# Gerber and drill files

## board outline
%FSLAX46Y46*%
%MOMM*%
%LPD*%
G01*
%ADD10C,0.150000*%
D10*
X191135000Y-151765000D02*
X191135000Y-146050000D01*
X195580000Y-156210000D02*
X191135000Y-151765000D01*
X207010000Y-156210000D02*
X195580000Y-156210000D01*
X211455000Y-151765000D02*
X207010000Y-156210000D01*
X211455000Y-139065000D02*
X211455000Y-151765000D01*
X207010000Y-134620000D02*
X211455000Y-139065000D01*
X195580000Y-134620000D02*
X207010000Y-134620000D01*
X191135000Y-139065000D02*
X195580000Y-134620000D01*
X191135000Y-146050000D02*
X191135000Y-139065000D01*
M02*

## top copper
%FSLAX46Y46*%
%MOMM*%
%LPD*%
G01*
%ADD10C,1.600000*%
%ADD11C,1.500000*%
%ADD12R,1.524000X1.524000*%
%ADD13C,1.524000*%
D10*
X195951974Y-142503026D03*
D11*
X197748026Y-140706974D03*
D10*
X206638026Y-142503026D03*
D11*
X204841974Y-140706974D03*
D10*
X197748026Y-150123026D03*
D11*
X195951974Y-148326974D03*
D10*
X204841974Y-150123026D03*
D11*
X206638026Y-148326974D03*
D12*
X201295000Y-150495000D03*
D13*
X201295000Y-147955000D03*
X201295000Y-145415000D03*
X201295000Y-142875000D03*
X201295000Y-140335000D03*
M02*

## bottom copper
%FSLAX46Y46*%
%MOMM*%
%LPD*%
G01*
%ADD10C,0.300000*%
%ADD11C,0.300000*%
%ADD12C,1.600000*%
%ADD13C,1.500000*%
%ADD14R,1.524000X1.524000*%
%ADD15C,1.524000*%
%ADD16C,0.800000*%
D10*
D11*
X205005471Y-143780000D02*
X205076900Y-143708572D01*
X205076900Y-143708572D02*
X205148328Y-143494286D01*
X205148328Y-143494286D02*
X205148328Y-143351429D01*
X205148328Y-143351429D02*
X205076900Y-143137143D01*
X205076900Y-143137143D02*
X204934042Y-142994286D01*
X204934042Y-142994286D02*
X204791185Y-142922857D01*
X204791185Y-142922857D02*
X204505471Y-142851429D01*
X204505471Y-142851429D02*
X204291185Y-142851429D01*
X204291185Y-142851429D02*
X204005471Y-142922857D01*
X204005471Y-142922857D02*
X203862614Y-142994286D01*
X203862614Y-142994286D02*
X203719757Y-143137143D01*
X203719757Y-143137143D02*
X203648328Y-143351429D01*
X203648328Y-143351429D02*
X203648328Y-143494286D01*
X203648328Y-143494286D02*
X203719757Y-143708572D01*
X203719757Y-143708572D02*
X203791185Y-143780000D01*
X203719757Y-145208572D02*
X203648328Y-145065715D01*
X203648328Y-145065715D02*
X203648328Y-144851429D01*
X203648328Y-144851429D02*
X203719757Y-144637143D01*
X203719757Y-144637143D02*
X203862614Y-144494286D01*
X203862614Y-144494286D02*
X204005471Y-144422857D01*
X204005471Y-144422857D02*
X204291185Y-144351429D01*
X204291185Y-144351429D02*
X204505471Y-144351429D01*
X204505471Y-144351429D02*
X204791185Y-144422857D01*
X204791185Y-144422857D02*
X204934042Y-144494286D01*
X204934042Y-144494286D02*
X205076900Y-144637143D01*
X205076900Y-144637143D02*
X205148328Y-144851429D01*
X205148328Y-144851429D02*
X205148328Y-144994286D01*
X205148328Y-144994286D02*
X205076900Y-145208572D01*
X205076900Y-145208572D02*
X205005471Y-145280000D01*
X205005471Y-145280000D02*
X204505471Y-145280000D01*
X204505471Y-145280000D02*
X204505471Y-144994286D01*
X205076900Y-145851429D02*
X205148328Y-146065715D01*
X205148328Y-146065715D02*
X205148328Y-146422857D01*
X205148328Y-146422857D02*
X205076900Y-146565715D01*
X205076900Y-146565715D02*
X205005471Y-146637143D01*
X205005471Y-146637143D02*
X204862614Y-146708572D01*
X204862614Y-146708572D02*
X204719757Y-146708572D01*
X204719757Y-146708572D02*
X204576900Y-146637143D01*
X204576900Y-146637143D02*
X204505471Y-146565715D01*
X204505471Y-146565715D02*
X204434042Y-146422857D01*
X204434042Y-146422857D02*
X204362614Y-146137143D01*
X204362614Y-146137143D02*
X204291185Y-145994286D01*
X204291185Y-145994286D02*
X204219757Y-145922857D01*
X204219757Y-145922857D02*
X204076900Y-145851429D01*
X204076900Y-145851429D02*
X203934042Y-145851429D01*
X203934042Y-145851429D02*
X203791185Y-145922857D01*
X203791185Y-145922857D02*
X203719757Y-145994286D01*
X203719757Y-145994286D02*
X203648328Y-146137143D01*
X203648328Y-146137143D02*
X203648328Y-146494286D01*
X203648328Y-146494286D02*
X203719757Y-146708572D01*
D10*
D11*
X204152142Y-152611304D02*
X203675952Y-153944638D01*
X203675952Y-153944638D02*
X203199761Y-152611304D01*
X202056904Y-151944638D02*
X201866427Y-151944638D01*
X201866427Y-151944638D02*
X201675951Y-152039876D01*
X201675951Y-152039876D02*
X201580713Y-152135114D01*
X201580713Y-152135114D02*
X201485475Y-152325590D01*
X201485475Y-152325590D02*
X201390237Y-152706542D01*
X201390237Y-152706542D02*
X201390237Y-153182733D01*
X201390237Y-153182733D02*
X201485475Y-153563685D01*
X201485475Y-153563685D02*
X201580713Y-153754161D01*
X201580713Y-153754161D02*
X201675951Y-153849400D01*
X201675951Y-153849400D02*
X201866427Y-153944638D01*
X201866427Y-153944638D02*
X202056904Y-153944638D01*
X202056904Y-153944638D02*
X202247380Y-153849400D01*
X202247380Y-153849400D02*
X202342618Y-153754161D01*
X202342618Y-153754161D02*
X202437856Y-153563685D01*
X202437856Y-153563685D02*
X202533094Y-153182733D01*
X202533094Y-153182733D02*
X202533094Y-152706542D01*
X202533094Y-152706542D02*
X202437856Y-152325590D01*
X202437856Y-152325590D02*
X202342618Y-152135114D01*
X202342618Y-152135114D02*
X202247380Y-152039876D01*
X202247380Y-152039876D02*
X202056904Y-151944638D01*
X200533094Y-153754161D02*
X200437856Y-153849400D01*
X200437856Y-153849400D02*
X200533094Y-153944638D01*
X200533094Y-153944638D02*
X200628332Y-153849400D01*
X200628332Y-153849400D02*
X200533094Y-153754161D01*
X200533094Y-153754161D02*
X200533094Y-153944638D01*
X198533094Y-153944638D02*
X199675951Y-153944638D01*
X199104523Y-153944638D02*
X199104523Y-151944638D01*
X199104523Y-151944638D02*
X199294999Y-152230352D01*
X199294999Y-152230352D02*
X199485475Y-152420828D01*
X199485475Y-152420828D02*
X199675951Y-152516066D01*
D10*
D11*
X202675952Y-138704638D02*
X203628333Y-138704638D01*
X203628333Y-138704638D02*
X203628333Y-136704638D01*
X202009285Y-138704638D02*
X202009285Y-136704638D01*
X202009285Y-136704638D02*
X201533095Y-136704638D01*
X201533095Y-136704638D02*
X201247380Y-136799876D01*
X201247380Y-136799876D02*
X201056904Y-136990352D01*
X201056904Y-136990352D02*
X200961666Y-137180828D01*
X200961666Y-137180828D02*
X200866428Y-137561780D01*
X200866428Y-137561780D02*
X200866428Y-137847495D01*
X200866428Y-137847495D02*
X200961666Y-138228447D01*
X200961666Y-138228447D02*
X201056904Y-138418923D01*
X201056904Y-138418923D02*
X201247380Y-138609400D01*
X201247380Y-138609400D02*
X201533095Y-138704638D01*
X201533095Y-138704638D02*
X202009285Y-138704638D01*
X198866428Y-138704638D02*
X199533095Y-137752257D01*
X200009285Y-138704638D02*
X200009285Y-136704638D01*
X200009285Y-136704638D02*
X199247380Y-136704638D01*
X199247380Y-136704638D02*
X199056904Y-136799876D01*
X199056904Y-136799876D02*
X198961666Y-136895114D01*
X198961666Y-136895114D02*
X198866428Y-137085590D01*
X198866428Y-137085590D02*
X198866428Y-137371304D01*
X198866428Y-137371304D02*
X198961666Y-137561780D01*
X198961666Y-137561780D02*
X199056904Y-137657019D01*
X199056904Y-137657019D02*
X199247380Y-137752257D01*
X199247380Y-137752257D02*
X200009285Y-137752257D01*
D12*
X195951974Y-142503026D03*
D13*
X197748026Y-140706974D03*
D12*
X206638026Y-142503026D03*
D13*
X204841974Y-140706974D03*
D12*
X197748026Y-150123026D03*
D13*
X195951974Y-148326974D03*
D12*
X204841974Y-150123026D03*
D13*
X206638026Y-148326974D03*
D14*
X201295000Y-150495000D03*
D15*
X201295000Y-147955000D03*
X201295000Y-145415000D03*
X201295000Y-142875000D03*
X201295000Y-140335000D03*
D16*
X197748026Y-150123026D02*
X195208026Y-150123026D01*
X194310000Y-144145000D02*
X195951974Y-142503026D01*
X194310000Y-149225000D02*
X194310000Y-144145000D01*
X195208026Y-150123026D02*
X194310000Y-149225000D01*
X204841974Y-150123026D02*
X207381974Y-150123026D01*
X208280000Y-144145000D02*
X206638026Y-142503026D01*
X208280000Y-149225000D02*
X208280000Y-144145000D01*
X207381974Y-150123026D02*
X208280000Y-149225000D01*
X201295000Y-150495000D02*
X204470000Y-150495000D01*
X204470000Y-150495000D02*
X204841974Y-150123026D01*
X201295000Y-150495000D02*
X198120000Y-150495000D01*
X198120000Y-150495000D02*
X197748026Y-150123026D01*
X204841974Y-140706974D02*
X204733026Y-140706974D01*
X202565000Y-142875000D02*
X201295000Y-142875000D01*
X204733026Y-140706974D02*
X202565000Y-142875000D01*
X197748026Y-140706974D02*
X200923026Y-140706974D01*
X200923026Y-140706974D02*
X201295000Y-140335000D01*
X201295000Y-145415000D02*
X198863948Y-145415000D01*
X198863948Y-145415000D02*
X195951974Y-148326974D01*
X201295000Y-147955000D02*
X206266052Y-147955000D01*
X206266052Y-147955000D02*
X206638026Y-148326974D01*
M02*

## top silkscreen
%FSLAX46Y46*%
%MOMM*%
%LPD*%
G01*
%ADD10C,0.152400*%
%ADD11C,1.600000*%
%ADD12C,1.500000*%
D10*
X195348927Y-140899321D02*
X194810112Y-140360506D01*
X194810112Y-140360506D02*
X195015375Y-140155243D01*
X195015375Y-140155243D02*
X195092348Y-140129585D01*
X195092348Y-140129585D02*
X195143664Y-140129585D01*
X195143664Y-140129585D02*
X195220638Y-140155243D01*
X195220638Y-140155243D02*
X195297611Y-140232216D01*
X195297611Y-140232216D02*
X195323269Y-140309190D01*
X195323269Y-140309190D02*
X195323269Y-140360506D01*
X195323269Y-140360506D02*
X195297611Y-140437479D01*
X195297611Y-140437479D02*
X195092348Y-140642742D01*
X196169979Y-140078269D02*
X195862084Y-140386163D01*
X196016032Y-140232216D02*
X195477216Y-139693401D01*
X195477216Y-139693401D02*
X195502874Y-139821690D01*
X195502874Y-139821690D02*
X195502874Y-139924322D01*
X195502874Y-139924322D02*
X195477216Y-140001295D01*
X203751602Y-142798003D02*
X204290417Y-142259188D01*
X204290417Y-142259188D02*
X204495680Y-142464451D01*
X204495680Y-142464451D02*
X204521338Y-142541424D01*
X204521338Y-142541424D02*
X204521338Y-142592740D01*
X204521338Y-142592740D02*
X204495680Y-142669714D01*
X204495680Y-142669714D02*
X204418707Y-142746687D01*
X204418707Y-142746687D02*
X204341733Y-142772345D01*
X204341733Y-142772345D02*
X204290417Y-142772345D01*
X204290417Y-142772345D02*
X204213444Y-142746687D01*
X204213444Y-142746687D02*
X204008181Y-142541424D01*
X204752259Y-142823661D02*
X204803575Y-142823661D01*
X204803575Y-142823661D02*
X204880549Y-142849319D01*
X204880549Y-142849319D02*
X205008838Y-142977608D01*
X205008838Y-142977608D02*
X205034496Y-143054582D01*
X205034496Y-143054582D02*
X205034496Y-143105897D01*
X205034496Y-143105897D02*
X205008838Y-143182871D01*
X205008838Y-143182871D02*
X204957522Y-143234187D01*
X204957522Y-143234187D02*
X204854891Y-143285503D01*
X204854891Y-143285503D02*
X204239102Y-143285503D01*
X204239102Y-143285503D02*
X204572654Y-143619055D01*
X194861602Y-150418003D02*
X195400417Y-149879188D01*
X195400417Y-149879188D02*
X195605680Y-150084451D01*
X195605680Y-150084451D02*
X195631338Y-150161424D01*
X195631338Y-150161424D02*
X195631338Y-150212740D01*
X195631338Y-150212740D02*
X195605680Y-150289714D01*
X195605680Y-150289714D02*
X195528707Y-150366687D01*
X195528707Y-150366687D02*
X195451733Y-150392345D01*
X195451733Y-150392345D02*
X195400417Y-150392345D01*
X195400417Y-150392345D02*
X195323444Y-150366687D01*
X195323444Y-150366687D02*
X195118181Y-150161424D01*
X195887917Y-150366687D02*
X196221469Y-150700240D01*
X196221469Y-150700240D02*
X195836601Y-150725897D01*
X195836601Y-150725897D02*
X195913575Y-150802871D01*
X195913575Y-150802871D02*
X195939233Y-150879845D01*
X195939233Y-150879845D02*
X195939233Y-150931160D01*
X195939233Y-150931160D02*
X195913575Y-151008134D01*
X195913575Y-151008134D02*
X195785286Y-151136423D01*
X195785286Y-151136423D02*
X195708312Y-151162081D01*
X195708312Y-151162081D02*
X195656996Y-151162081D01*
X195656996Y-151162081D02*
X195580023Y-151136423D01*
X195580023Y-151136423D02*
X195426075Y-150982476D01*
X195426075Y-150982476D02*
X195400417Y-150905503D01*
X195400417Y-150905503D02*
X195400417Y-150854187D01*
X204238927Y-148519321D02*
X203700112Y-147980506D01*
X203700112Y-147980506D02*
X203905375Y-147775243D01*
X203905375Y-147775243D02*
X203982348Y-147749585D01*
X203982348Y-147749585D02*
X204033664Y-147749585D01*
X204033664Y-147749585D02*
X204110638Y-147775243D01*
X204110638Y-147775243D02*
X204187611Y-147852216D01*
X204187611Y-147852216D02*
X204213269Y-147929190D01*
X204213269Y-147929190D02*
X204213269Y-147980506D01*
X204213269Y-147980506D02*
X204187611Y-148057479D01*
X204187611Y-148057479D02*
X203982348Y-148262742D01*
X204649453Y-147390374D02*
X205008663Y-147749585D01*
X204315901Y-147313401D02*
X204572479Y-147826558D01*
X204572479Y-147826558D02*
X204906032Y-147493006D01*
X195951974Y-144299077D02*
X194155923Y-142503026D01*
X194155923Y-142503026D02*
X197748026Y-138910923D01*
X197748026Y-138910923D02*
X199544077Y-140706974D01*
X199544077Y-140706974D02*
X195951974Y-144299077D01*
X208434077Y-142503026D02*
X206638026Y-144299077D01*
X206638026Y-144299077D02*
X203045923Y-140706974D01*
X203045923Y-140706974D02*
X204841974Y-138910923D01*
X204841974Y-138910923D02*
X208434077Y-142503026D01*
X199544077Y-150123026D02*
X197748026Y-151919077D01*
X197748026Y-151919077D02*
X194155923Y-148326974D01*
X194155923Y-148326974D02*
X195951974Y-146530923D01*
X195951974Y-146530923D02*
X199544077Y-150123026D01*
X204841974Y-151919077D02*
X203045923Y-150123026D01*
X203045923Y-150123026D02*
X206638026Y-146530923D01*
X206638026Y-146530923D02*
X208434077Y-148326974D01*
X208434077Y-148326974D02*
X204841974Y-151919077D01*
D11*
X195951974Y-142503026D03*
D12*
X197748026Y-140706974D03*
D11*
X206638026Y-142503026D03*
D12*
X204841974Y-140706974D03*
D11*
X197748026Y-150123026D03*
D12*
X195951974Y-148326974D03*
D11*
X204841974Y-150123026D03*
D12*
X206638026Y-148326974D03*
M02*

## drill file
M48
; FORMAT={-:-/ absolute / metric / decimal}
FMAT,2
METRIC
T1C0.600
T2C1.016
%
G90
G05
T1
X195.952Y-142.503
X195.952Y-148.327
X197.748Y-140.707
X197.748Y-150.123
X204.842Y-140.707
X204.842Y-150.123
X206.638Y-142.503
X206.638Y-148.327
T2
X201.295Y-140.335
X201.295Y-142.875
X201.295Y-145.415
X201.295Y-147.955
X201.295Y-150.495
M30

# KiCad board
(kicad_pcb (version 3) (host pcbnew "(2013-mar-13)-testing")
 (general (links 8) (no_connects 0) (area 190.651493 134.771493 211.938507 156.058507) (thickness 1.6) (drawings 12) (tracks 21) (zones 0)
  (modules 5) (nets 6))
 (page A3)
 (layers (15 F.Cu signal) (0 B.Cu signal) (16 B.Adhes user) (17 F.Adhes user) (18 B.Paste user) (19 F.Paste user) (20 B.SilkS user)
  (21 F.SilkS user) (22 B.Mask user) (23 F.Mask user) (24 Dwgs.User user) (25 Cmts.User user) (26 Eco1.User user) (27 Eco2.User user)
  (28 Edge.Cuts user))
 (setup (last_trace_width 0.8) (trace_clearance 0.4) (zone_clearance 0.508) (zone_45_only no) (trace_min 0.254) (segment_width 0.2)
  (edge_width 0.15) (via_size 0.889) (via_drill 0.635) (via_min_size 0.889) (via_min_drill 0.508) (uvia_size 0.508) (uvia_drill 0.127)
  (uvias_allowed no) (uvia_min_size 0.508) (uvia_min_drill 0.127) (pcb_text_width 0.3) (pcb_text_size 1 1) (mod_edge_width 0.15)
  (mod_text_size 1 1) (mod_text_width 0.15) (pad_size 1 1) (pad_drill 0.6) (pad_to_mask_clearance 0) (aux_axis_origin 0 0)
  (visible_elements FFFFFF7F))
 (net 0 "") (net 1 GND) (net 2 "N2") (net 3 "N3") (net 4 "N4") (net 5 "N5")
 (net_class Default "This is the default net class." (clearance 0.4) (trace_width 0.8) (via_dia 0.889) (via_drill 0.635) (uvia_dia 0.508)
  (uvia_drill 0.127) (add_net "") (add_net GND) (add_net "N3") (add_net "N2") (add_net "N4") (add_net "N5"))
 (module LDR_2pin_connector (layer F.Cu) (at 196.85 141.605 45)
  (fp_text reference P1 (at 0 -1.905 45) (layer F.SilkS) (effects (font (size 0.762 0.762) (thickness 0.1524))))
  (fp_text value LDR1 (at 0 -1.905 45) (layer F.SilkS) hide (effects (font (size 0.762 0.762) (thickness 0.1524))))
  (fp_line (start -2.54 1.27) (end -2.54 -1.27) (layer F.SilkS) (width 0.1524))
  (fp_line (start -2.54 -1.27) (end 2.54 -1.27) (layer F.SilkS) (width 0.1524))
  (fp_line (start 2.54 -1.27) (end 2.54 1.27) (layer F.SilkS) (width 0.1524))
  (fp_line (start 2.54 1.27) (end -2.54 1.27) (layer F.SilkS) (width 0.1524))
  (pad 1 thru_hole circle (at -1.27 0 45) (size 1.6 1.6) (drill 0.6) (layers *.Cu *.Mask F.SilkS) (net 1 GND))
  (pad 2 thru_hole circle (at 1.27 0 45) (size 1.5 1.5) (drill 0.6) (layers *.Cu *.Mask F.SilkS) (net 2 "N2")))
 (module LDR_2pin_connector (layer F.Cu) (at 205.74 141.605 135)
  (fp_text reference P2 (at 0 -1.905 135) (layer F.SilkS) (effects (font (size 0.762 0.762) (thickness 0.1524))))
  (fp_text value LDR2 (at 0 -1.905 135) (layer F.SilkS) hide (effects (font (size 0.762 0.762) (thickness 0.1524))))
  (fp_line (start -2.54 1.27) (end -2.54 -1.27) (layer F.SilkS) (width 0.1524))
  (fp_line (start -2.54 -1.27) (end 2.54 -1.27) (layer F.SilkS) (width 0.1524))
  (fp_line (start 2.54 -1.27) (end 2.54 1.27) (layer F.SilkS) (width 0.1524))
  (fp_line (start 2.54 1.27) (end -2.54 1.27) (layer F.SilkS) (width 0.1524))
  (pad 1 thru_hole circle (at -1.27 0 135) (size 1.6 1.6) (drill 0.6) (layers *.Cu *.Mask F.SilkS) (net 1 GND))
  (pad 2 thru_hole circle (at 1.27 0 135) (size 1.5 1.5) (drill 0.6) (layers *.Cu *.Mask F.SilkS) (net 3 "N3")))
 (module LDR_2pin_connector (layer F.Cu) (at 196.85 149.225 135)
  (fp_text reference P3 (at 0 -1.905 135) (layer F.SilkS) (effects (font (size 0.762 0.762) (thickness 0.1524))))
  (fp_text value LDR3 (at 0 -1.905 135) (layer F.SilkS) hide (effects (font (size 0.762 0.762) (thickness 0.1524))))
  (fp_line (start -2.54 1.27) (end -2.54 -1.27) (layer F.SilkS) (width 0.1524))
  (fp_line (start -2.54 -1.27) (end 2.54 -1.27) (layer F.SilkS) (width 0.1524))
  (fp_line (start 2.54 -1.27) (end 2.54 1.27) (layer F.SilkS) (width 0.1524))
  (fp_line (start 2.54 1.27) (end -2.54 1.27) (layer F.SilkS) (width 0.1524))
  (pad 1 thru_hole circle (at -1.27 0 135) (size 1.6 1.6) (drill 0.6) (layers *.Cu *.Mask F.SilkS) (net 1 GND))
  (pad 2 thru_hole circle (at 1.27 0 135) (size 1.5 1.5) (drill 0.6) (layers *.Cu *.Mask F.SilkS) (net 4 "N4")))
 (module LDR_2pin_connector (layer F.Cu) (at 205.74 149.225 45)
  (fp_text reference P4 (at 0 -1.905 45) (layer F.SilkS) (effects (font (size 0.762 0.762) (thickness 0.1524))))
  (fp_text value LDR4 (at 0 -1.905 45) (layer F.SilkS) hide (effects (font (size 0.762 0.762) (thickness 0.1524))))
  (fp_line (start -2.54 1.27) (end -2.54 -1.27) (layer F.SilkS) (width 0.1524))
  (fp_line (start -2.54 -1.27) (end 2.54 -1.27) (layer F.SilkS) (width 0.1524))
  (fp_line (start 2.54 -1.27) (end 2.54 1.27) (layer F.SilkS) (width 0.1524))
  (fp_line (start 2.54 1.27) (end -2.54 1.27) (layer F.SilkS) (width 0.1524))
  (pad 1 thru_hole circle (at -1.27 0 45) (size 1.6 1.6) (drill 0.6) (layers *.Cu *.Mask F.SilkS) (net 1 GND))
  (pad 2 thru_hole circle (at 1.27 0 45) (size 1.5 1.5) (drill 0.6) (layers *.Cu *.Mask F.SilkS) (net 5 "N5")))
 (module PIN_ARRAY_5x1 (layer B.Cu) (at 201.295 145.415 90)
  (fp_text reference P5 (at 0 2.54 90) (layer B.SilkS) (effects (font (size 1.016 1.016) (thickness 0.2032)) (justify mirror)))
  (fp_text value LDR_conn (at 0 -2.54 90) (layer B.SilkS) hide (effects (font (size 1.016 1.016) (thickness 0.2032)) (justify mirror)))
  (pad 1 thru_hole rect (at -5.08 0 90) (size 1.524 1.524) (drill 1.016) (layers *.Cu *.Mask B.SilkS) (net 1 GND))
  (pad 2 thru_hole circle (at -2.54 0 90) (size 1.524 1.524) (drill 1.016) (layers *.Cu *.Mask B.SilkS) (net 5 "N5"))
  (pad 3 thru_hole circle (at 0 0 90) (size 1.524 1.524) (drill 1.016) (layers *.Cu *.Mask B.SilkS) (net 4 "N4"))
  (pad 4 thru_hole circle (at 2.54 0 90) (size 1.524 1.524) (drill 1.016) (layers *.Cu *.Mask B.SilkS) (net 3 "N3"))
  (pad 5 thru_hole circle (at 5.08 0 90) (size 1.524 1.524) (drill 1.016) (layers *.Cu *.Mask B.SilkS) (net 2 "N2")))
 (gr_line (start 191.135 151.765) (end 191.135 146.05) (angle 90) (layer Edge.Cuts) (width 0.15))
 (gr_line (start 195.58 156.21) (end 191.135 151.765) (angle 90) (layer Edge.Cuts) (width 0.15))
 (gr_line (start 207.01 156.21) (end 195.58 156.21) (angle 90) (layer Edge.Cuts) (width 0.15))
 (gr_line (start 211.455 151.765) (end 207.01 156.21) (angle 90) (layer Edge.Cuts) (width 0.15))
 (gr_line (start 211.455 139.065) (end 211.455 151.765) (angle 90) (layer Edge.Cuts) (width 0.15))
 (gr_line (start 207.01 134.62) (end 211.455 139.065) (angle 90) (layer Edge.Cuts) (width 0.15))
 (gr_line (start 195.58 134.62) (end 207.01 134.62) (angle 90) (layer Edge.Cuts) (width 0.15))
 (gr_line (start 191.135 139.065) (end 195.58 134.62) (angle 90) (layer Edge.Cuts) (width 0.15))
 (gr_line (start 191.135 146.05) (end 191.135 139.065) (angle 90) (layer Edge.Cuts) (width 0.15))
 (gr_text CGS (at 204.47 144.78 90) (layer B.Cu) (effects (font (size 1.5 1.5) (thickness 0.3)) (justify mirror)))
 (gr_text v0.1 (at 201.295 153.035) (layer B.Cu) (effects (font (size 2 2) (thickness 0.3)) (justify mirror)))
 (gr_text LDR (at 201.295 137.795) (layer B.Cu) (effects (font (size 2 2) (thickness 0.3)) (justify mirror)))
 (segment (start 197.748026 150.123026) (end 195.208026 150.123026) (width 0.8) (layer B.Cu) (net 1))
 (segment (start 194.31 144.145) (end 195.951974 142.503026) (width 0.8) (layer B.Cu) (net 1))
 (segment (start 194.31 149.225) (end 194.31 144.145) (width 0.8) (layer B.Cu) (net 1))
 (segment (start 195.208026 150.123026) (end 194.31 149.225) (width 0.8) (layer B.Cu) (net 1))
 (segment (start 204.841974 150.123026) (end 207.381974 150.123026) (width 0.8) (layer B.Cu) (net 1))
 (segment (start 208.28 144.145) (end 206.638026 142.503026) (width 0.8) (layer B.Cu) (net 1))
 (segment (start 208.28 149.225) (end 208.28 144.145) (width 0.8) (layer B.Cu) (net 1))
 (segment (start 207.381974 150.123026) (end 208.28 149.225) (width 0.8) (layer B.Cu) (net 1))
 (segment (start 201.295 150.495) (end 204.47 150.495) (width 0.8) (layer B.Cu) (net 1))
 (segment (start 204.47 150.495) (end 204.841974 150.123026) (width 0.8) (layer B.Cu) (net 1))
 (segment (start 201.295 150.495) (end 198.12 150.495) (width 0.8) (layer B.Cu) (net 1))
 (segment (start 198.12 150.495) (end 197.748026 150.123026) (width 0.8) (layer B.Cu) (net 1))
 (segment (start 204.841974 140.706974) (end 204.733026 140.706974) (width 0.8) (layer B.Cu) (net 3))
 (segment (start 202.565 142.875) (end 201.295 142.875) (width 0.8) (layer B.Cu) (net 3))
 (segment (start 204.733026 140.706974) (end 202.565 142.875) (width 0.8) (layer B.Cu) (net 3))
 (segment (start 197.748026 140.706974) (end 200.923026 140.706974) (width 0.8) (layer B.Cu) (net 2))
 (segment (start 200.923026 140.706974) (end 201.295 140.335) (width 0.8) (layer B.Cu) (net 2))
 (segment (start 201.295 145.415) (end 198.863948 145.415) (width 0.8) (layer B.Cu) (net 4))
 (segment (start 198.863948 145.415) (end 195.951974 148.326974) (width 0.8) (layer B.Cu) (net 4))
 (segment (start 201.295 147.955) (end 206.266052 147.955) (width 0.8) (layer B.Cu) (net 5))
 (segment (start 206.266052 147.955) (end 206.638026 148.326974) (width 0.8) (layer B.Cu) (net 5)))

